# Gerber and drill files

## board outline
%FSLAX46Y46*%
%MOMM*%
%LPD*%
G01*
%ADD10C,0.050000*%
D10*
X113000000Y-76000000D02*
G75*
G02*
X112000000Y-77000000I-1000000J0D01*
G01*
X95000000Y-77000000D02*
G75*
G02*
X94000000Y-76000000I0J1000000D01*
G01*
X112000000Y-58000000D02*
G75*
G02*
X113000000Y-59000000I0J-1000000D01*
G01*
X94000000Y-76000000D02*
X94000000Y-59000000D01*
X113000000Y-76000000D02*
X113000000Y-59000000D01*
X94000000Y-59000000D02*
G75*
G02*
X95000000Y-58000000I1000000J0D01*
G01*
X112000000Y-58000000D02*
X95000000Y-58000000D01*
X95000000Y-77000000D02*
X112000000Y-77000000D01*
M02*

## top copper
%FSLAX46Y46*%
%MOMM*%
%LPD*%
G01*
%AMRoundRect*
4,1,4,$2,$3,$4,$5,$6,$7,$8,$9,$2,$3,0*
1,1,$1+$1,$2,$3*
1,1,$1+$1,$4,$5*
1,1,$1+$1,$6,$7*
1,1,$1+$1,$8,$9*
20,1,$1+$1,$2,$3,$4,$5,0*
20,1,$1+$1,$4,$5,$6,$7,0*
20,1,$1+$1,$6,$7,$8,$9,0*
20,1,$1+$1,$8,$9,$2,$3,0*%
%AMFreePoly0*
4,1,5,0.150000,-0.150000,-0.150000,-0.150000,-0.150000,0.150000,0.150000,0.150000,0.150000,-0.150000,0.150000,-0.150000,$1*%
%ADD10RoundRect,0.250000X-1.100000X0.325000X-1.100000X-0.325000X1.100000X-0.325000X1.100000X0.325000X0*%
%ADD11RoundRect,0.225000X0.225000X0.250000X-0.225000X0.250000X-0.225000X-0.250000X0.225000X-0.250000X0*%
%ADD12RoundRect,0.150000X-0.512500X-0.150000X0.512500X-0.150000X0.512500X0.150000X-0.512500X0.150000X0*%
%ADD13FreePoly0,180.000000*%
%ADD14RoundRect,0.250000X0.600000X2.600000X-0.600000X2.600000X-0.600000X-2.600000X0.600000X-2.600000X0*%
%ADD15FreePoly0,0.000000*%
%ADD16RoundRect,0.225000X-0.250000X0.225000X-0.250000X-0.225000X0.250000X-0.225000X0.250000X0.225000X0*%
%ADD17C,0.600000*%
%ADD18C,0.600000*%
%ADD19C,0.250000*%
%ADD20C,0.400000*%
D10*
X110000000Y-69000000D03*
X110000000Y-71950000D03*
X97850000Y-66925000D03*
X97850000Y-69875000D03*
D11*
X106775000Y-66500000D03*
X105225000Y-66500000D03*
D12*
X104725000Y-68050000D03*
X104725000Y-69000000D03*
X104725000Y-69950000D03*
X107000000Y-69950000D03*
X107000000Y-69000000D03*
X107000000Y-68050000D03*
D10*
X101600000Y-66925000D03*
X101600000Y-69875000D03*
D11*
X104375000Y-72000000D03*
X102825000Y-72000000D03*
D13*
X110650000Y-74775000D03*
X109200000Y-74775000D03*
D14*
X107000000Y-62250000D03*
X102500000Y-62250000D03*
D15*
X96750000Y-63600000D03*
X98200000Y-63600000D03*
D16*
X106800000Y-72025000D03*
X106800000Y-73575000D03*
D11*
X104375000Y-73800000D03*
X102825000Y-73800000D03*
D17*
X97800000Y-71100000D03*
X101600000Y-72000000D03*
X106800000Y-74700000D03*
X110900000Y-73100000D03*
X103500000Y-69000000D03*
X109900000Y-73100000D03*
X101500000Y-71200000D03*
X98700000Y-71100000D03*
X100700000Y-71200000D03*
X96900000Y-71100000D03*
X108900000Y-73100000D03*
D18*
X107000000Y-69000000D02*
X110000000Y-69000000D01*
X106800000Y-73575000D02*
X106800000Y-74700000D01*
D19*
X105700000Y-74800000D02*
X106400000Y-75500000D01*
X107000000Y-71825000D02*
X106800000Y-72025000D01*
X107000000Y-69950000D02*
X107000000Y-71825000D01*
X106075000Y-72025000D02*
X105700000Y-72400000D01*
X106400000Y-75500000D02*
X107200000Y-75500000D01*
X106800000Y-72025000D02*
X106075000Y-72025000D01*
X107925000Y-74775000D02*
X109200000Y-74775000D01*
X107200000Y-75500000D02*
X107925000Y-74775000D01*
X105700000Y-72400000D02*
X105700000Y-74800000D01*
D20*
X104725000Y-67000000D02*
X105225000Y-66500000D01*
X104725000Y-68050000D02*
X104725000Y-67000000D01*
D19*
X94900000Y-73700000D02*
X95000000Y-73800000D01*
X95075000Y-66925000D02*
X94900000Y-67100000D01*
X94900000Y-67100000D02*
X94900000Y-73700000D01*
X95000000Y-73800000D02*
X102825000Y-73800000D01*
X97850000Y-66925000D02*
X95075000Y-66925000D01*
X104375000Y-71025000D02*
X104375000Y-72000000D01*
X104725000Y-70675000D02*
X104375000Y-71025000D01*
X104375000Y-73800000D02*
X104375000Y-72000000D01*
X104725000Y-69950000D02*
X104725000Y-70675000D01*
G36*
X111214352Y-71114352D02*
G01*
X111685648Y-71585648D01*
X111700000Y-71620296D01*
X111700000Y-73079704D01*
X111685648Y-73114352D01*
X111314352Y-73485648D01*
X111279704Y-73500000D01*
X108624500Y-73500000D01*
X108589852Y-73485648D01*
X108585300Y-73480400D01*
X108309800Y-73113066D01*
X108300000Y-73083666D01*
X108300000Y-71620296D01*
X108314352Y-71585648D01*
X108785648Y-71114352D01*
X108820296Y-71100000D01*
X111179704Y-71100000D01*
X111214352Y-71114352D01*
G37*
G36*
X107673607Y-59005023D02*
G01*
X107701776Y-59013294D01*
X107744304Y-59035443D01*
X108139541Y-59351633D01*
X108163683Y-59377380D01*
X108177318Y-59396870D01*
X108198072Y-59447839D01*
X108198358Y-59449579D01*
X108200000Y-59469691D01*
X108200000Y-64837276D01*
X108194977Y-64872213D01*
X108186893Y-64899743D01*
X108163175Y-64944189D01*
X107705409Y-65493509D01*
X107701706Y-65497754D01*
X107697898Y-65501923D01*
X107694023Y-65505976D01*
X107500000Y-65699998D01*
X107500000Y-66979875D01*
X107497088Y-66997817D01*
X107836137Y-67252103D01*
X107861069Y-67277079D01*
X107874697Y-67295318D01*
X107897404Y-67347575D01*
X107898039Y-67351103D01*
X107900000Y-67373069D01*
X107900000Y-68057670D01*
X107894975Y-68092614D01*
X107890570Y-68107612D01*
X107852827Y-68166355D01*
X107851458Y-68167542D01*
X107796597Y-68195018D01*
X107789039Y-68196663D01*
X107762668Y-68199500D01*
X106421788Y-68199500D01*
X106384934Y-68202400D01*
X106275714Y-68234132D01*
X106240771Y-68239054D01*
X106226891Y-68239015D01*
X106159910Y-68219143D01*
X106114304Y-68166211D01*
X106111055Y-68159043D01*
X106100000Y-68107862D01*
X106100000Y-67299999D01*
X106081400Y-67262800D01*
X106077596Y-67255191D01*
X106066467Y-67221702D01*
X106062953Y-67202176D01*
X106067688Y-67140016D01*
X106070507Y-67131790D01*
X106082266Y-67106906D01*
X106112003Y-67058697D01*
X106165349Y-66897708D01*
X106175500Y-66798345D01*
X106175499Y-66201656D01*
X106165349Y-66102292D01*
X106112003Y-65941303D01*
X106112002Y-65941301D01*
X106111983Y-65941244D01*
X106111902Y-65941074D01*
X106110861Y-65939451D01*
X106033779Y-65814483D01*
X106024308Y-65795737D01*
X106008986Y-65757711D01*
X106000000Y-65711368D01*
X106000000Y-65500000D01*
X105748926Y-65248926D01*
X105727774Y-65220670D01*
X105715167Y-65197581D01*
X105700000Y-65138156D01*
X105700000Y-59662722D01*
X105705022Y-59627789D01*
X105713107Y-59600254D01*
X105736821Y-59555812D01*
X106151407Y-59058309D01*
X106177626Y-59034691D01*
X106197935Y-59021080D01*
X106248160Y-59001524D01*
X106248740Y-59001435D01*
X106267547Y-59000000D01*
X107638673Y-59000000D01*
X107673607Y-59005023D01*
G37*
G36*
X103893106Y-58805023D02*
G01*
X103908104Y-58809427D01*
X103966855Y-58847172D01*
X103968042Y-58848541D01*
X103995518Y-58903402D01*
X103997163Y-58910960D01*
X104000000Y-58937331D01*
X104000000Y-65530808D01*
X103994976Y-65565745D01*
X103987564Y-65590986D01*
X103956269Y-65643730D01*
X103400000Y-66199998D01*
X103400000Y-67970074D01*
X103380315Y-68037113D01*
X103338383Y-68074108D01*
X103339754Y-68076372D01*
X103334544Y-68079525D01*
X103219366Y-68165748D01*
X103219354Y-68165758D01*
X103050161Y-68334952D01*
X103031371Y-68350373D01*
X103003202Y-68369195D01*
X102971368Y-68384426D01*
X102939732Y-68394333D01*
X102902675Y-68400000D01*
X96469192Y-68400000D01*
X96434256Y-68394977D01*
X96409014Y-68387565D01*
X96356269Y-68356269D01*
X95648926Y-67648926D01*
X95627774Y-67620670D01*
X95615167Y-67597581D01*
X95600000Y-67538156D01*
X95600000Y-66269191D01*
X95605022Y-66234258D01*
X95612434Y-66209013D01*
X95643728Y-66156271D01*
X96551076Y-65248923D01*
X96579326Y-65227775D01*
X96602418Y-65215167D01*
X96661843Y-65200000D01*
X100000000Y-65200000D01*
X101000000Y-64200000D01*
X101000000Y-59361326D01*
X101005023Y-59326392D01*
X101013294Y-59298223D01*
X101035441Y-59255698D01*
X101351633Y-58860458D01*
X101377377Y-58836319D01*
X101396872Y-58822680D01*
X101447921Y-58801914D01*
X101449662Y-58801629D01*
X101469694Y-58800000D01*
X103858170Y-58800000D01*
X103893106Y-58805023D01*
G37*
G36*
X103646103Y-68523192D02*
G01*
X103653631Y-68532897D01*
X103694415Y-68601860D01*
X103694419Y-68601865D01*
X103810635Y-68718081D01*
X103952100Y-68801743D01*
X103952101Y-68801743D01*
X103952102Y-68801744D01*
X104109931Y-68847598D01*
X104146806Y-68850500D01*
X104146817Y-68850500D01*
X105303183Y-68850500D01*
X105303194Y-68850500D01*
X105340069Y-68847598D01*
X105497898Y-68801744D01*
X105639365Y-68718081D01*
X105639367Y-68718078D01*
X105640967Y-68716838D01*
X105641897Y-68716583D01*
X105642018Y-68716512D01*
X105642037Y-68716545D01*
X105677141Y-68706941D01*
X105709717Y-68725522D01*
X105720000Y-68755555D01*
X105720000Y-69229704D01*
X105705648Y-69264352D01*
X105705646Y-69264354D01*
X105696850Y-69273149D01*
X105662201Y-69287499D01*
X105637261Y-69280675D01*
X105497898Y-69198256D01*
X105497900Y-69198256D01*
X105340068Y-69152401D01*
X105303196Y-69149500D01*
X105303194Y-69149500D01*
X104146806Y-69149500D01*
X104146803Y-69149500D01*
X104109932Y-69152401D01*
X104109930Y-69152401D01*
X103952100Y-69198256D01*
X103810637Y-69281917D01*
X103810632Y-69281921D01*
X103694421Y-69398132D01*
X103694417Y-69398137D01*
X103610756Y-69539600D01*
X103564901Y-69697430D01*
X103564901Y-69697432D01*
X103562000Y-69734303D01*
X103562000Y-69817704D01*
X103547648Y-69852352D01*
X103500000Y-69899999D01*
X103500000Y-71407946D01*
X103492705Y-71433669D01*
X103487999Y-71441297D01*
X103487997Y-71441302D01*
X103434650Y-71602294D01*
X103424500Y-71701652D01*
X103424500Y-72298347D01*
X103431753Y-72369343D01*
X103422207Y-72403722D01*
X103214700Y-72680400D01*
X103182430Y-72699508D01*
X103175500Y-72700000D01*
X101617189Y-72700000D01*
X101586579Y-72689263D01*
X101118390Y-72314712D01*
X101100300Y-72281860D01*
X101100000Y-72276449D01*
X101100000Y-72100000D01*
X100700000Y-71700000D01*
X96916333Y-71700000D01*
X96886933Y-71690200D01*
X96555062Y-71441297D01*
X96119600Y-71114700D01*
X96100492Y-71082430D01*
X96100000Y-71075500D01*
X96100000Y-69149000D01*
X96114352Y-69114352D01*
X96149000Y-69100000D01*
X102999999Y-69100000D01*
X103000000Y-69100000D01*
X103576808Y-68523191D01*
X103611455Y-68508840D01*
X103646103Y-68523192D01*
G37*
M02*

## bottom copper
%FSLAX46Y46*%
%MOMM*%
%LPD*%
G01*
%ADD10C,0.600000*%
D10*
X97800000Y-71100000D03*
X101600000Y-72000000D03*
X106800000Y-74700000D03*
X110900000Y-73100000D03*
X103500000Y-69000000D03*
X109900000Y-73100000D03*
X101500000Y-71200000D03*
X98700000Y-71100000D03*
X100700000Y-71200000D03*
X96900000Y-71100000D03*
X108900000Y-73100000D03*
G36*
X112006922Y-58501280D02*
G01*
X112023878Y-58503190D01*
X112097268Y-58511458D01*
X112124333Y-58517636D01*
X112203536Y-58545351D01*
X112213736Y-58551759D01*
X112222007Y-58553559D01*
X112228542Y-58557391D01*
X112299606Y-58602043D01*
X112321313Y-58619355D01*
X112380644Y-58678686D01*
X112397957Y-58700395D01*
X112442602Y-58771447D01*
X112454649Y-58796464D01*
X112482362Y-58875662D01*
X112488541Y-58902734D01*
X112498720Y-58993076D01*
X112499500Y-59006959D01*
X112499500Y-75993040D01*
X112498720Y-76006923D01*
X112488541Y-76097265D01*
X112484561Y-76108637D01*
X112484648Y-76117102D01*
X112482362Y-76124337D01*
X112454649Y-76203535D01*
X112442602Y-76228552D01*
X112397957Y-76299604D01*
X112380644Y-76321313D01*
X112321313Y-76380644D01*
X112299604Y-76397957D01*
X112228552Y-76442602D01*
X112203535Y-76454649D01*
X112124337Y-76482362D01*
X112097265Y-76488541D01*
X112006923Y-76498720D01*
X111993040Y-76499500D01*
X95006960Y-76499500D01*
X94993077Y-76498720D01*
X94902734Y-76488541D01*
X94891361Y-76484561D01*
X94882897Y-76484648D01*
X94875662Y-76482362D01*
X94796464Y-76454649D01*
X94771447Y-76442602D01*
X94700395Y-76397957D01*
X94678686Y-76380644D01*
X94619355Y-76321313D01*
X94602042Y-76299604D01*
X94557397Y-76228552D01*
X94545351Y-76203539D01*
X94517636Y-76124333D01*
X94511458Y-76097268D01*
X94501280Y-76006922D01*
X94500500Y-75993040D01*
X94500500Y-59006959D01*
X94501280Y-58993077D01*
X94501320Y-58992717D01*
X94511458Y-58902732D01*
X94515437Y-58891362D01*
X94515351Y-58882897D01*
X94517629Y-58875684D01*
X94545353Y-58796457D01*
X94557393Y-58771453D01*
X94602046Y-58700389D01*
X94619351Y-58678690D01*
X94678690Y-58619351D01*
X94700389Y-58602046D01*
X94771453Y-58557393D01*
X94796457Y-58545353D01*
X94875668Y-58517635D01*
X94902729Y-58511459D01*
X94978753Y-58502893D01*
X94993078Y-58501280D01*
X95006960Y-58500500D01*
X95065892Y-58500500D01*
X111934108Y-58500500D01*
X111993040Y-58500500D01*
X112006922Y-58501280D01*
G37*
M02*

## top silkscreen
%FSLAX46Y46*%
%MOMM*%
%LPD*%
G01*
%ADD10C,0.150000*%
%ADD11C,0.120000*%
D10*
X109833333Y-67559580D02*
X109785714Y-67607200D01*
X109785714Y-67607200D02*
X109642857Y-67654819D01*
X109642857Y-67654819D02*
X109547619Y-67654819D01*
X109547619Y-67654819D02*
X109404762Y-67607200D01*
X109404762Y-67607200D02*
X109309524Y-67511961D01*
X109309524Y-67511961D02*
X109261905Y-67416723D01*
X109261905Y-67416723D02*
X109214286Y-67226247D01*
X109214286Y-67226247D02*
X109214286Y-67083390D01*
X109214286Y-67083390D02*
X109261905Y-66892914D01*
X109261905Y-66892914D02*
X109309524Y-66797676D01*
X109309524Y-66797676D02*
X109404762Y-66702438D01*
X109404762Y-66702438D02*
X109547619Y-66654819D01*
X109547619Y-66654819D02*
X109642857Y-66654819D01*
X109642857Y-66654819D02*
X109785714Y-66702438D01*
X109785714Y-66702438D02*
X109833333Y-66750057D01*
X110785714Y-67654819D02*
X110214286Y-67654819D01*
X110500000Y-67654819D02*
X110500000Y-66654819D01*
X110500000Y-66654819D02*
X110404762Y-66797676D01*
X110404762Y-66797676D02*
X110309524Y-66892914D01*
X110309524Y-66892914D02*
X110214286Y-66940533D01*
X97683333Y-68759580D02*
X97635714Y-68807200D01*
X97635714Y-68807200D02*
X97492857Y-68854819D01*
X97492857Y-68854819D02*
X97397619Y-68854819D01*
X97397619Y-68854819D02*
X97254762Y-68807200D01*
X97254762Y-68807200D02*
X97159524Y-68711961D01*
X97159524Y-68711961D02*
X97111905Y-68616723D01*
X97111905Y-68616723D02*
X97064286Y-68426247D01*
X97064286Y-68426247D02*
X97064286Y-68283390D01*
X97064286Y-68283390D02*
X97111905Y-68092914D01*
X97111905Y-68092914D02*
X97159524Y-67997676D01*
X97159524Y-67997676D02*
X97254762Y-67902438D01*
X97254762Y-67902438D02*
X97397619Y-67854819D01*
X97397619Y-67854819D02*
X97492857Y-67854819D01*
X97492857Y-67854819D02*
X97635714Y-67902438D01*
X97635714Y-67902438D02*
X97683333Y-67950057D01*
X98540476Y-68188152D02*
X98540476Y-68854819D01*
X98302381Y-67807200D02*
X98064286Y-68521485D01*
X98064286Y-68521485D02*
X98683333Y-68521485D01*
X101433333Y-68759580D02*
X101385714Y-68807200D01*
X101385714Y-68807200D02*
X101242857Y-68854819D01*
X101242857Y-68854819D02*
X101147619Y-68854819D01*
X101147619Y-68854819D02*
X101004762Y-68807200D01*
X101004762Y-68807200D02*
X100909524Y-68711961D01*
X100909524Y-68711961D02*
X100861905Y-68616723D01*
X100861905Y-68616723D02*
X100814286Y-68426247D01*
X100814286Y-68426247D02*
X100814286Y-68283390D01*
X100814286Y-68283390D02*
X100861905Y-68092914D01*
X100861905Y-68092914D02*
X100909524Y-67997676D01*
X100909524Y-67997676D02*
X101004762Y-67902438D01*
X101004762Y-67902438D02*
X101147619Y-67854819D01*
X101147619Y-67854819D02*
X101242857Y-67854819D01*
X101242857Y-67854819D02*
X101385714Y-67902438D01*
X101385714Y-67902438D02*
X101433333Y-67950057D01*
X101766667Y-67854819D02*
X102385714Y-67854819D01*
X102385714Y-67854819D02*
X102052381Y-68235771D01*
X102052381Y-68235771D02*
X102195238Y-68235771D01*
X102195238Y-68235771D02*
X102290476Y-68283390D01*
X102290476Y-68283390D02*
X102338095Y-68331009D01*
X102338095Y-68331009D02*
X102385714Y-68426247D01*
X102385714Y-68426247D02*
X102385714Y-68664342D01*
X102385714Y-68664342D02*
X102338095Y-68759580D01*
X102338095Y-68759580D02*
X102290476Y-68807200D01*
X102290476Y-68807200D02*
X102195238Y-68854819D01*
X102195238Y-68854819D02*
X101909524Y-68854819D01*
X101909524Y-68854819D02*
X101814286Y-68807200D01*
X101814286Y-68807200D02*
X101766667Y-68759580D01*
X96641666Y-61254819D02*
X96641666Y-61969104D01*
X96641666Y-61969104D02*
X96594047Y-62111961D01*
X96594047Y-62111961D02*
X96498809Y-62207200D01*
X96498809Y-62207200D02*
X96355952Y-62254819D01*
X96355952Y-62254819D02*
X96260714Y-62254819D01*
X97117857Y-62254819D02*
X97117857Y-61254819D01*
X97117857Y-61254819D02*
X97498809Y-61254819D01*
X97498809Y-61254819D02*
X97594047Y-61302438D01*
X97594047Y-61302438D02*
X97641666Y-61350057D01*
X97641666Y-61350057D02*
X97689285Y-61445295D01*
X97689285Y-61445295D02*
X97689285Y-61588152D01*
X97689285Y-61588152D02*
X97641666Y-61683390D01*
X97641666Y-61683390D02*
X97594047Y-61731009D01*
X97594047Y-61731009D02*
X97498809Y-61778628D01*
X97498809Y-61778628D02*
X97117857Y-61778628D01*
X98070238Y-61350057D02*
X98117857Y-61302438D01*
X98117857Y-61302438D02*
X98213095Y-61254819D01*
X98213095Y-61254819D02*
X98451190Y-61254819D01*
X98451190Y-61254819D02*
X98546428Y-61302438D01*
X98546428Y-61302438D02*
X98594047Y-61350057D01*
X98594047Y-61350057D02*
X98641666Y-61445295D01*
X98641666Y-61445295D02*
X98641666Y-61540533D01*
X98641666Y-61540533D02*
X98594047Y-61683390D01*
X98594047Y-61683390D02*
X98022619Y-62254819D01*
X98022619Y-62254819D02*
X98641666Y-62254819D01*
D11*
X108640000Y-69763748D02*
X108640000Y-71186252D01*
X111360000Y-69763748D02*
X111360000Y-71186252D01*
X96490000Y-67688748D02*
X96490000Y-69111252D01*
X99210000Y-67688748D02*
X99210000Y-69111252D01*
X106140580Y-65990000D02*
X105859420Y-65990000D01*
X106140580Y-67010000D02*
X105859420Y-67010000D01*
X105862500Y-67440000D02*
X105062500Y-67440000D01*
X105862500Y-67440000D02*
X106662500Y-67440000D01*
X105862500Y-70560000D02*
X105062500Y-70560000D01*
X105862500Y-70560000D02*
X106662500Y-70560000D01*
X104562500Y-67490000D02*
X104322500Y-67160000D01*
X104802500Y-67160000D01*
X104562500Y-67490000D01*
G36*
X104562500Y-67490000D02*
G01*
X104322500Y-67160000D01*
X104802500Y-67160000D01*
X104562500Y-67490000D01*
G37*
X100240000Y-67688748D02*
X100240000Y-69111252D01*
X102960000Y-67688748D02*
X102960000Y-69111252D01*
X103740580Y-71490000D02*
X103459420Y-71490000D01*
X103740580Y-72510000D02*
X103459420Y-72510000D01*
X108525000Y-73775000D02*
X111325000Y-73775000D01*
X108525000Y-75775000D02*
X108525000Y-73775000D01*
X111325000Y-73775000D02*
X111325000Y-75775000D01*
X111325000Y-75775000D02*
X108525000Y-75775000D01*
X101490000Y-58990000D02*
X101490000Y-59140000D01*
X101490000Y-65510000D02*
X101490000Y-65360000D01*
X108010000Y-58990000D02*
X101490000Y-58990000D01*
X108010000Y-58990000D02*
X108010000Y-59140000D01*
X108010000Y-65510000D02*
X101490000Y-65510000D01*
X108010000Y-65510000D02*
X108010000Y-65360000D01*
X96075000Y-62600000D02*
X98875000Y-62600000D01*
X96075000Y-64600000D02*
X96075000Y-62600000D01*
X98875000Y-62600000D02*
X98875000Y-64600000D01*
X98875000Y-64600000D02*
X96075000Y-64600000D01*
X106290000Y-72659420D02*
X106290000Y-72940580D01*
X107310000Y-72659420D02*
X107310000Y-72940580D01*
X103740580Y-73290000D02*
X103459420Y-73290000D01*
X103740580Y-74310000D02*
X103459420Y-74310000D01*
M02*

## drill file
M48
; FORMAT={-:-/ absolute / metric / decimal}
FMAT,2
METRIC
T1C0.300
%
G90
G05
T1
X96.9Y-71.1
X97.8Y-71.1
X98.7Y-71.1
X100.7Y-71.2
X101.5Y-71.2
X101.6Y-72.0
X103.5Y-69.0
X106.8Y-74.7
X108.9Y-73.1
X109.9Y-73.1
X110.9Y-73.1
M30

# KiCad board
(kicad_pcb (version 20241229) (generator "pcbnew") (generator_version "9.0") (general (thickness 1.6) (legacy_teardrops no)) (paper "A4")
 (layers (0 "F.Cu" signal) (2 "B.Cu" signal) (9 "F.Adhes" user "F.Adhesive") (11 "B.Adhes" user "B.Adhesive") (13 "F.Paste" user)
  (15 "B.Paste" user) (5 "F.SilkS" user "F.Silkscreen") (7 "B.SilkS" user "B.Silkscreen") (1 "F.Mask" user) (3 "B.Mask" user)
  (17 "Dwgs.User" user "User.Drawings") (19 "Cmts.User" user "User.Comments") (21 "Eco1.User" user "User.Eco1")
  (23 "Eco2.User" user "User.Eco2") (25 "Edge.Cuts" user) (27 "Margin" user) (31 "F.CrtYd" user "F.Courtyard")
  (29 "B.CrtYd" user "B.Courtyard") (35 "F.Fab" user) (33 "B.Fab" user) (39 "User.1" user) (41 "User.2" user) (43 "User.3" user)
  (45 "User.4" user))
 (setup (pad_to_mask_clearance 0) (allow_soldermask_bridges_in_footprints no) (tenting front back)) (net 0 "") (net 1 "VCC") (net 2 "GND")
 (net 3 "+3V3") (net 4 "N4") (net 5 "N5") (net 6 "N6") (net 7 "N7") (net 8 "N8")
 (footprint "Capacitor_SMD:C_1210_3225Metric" (layer "F.Cu") (at 110 70.475 -90)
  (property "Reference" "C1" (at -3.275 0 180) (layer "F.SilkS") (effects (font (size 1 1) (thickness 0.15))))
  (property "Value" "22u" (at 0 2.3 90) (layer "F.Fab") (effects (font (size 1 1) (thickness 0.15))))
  (fp_line (start -0.711252 1.36) (end 0.711252 1.36) (stroke (width 0.12) (type solid)) (layer "F.SilkS"))
  (fp_line (start -0.711252 -1.36) (end 0.711252 -1.36) (stroke (width 0.12) (type solid)) (layer "F.SilkS"))
  (pad "1" smd roundrect (at -1.475 0 270) (size 1.15 2.7) (layers "F.Cu" "F.Mask" "F.Paste") (roundrect_rratio 0.217391) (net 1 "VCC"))
  (pad "2" smd roundrect (at 1.475 0 270) (size 1.15 2.7) (layers "F.Cu" "F.Mask" "F.Paste") (roundrect_rratio 0.217391) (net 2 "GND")))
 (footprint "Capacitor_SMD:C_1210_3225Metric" (layer "F.Cu") (at 97.85 68.4 -90)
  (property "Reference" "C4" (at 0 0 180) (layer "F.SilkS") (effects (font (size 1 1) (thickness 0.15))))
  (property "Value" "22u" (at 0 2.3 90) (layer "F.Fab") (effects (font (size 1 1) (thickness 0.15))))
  (fp_line (start -0.711252 1.36) (end 0.711252 1.36) (stroke (width 0.12) (type solid)) (layer "F.SilkS"))
  (fp_line (start -0.711252 -1.36) (end 0.711252 -1.36) (stroke (width 0.12) (type solid)) (layer "F.SilkS"))
  (pad "1" smd roundrect (at -1.475 0 270) (size 1.15 2.7) (layers "F.Cu" "F.Mask" "F.Paste") (roundrect_rratio 0.217391) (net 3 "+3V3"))
  (pad "2" smd roundrect (at 1.475 0 270) (size 1.15 2.7) (layers "F.Cu" "F.Mask" "F.Paste") (roundrect_rratio 0.217391) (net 2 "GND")))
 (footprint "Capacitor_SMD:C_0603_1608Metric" (layer "F.Cu") (at 106 66.5 180)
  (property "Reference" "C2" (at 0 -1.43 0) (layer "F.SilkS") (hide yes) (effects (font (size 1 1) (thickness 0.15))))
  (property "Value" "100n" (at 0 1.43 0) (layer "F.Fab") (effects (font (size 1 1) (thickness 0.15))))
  (fp_line (start -0.14058 0.51) (end 0.14058 0.51) (stroke (width 0.12) (type solid)) (layer "F.SilkS"))
  (fp_line (start -0.14058 -0.51) (end 0.14058 -0.51) (stroke (width 0.12) (type solid)) (layer "F.SilkS"))
  (pad "1" smd roundrect (at -0.775 0 180) (size 0.9 0.95) (layers "F.Cu" "F.Mask" "F.Paste") (roundrect_rratio 0.25) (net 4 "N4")
   (thermal_bridge_width 0.3) (thermal_gap 0.3))
  (pad "2" smd roundrect (at 0.775 0 180) (size 0.9 0.95) (layers "F.Cu" "F.Mask" "F.Paste") (roundrect_rratio 0.25) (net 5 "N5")))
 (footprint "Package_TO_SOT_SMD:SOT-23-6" (layer "F.Cu") (at 105.8625 69)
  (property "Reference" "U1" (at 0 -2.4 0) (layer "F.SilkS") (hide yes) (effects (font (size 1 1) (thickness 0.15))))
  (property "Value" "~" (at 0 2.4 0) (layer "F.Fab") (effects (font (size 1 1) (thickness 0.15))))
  (fp_line (start 0 -1.56) (end -0.8 -1.56) (stroke (width 0.12) (type solid)) (layer "F.SilkS"))
  (fp_line (start 0 -1.56) (end 0.8 -1.56) (stroke (width 0.12) (type solid)) (layer "F.SilkS"))
  (fp_line (start 0 1.56) (end -0.8 1.56) (stroke (width 0.12) (type solid)) (layer "F.SilkS"))
  (fp_line (start 0 1.56) (end 0.8 1.56) (stroke (width 0.12) (type solid)) (layer "F.SilkS"))
  (fp_poly
   (pts (xy -1.3 -1.51) (xy -1.54 -1.84) (xy -1.06 -1.84) (xy -1.3 -1.51)) (stroke (width 0.12) (type solid)) (fill yes) (layer "F.SilkS"))
  (pad "1" smd roundrect (at -1.1375 -0.95) (size 1.325 0.6) (layers "F.Cu" "F.Mask" "F.Paste") (roundrect_rratio 0.25) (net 5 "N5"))
  (pad "2" smd roundrect (at -1.1375 0) (size 1.325 0.6) (layers "F.Cu" "F.Mask" "F.Paste") (roundrect_rratio 0.25) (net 2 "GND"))
  (pad "3" smd roundrect (at -1.1375 0.95) (size 1.325 0.6) (layers "F.Cu" "F.Mask" "F.Paste") (roundrect_rratio 0.25) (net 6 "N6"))
  (pad "4" smd roundrect (at 1.1375 0.95) (size 1.325 0.6) (layers "F.Cu" "F.Mask" "F.Paste") (roundrect_rratio 0.25) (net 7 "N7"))
  (pad "5" smd roundrect (at 1.1375 0) (size 1.325 0.6) (layers "F.Cu" "F.Mask" "F.Paste") (roundrect_rratio 0.25) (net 1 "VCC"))
  (pad "6" smd roundrect (at 1.1375 -0.95) (size 1.325 0.6) (layers "F.Cu" "F.Mask" "F.Paste") (roundrect_rratio 0.25) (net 4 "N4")))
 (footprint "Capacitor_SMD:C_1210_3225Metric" (layer "F.Cu") (at 101.6 68.4 -90)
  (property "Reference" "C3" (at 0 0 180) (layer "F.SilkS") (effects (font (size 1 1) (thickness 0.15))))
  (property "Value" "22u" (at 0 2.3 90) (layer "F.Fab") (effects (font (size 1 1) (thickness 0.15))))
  (fp_line (start -0.711252 1.36) (end 0.711252 1.36) (stroke (width 0.12) (type solid)) (layer "F.SilkS"))
  (fp_line (start -0.711252 -1.36) (end 0.711252 -1.36) (stroke (width 0.12) (type solid)) (layer "F.SilkS"))
  (pad "1" smd roundrect (at -1.475 0 270) (size 1.15 2.7) (layers "F.Cu" "F.Mask" "F.Paste") (roundrect_rratio 0.217391) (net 3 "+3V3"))
  (pad "2" smd roundrect (at 1.475 0 270) (size 1.15 2.7) (layers "F.Cu" "F.Mask" "F.Paste") (roundrect_rratio 0.217391) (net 2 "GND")))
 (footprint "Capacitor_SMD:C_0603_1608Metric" (layer "F.Cu") (at 103.6 72 180)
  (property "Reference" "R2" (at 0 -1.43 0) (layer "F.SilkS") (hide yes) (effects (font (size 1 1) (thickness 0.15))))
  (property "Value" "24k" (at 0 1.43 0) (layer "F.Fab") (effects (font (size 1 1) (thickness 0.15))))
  (fp_line (start -0.14058 0.51) (end 0.14058 0.51) (stroke (width 0.12) (type solid)) (layer "F.SilkS"))
  (fp_line (start -0.14058 -0.51) (end 0.14058 -0.51) (stroke (width 0.12) (type solid)) (layer "F.SilkS"))
  (pad "1" smd roundrect (at -0.775 0 180) (size 0.9 0.95) (layers "F.Cu" "F.Mask" "F.Paste") (roundrect_rratio 0.25) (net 6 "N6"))
  (pad "2" smd roundrect (at 0.775 0 180) (size 0.9 0.95) (layers "F.Cu" "F.Mask" "F.Paste") (roundrect_rratio 0.25) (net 2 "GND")
   (thermal_bridge_width 0.2) (thermal_gap 0.2)))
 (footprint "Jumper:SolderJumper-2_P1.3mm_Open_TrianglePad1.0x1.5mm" (layer "F.Cu") (at 109.925 74.775 180)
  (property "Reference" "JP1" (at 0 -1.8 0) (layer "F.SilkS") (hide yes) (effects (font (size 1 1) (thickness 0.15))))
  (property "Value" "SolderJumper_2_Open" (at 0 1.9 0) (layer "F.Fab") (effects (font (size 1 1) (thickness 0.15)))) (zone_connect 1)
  (fp_line (start 1.4 1) (end -1.4 1) (stroke (width 0.12) (type solid)) (layer "F.SilkS"))
  (fp_line (start 1.4 -1) (end 1.4 1) (stroke (width 0.12) (type solid)) (layer "F.SilkS"))
  (fp_line (start -1.4 1) (end -1.4 -1) (stroke (width 0.12) (type solid)) (layer "F.SilkS"))
  (fp_line (start -1.4 -1) (end 1.4 -1) (stroke (width 0.12) (type solid)) (layer "F.SilkS"))
  (pad "1" smd custom (at -0.725 0 180) (size 0.3 0.3) (layers "F.Cu" "F.Mask") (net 1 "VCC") (zone_connect 2) (thermal_bridge_angle 45)
   (options (clearance outline) (anchor rect)) (primitives))
  (pad "2" smd custom (at 0.725 0 180) (size 0.3 0.3) (layers "F.Cu" "F.Mask") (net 7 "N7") (zone_connect 2) (thermal_bridge_angle 45)
   (options (clearance outline) (anchor rect)) (primitives)))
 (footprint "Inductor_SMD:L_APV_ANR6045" (layer "F.Cu") (at 104.75 62.25 180)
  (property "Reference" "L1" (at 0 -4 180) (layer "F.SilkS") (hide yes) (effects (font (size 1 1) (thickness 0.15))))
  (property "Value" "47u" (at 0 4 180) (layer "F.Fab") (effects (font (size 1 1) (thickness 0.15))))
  (fp_line (start 3.26 3.26) (end 3.26 3.11) (stroke (width 0.12) (type solid)) (layer "F.SilkS"))
  (fp_line (start 3.26 -3.26) (end 3.26 -3.11) (stroke (width 0.12) (type solid)) (layer "F.SilkS"))
  (fp_line (start -3.26 3.26) (end 3.26 3.26) (stroke (width 0.12) (type solid)) (layer "F.SilkS"))
  (fp_line (start -3.26 3.26) (end -3.26 3.11) (stroke (width 0.12) (type solid)) (layer "F.SilkS"))
  (fp_line (start -3.26 -3.26) (end 3.26 -3.26) (stroke (width 0.12) (type solid)) (layer "F.SilkS"))
  (fp_line (start -3.26 -3.26) (end -3.26 -3.11) (stroke (width 0.12) (type solid)) (layer "F.SilkS"))
  (pad "1" smd roundrect (at -2.25 0 180) (size 1.7 5.7) (layers "F.Cu" "F.Mask" "F.Paste") (roundrect_rratio 0.147059) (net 4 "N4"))
  (pad "2" smd roundrect (at 2.25 0 180) (size 1.7 5.7) (layers "F.Cu" "F.Mask" "F.Paste") (roundrect_rratio 0.147059) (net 3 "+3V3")))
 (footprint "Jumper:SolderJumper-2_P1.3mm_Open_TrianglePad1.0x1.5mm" (layer "F.Cu") (at 97.475 63.6)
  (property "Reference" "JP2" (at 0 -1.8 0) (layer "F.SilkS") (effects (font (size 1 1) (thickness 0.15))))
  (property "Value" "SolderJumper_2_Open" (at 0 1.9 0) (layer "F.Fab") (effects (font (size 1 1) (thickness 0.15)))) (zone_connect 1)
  (fp_line (start -1.4 -1) (end 1.4 -1) (stroke (width 0.12) (type solid)) (layer "F.SilkS"))
  (fp_line (start -1.4 1) (end -1.4 -1) (stroke (width 0.12) (type solid)) (layer "F.SilkS"))
  (fp_line (start 1.4 -1) (end 1.4 1) (stroke (width 0.12) (type solid)) (layer "F.SilkS"))
  (fp_line (start 1.4 1) (end -1.4 1) (stroke (width 0.12) (type solid)) (layer "F.SilkS"))
  (pad "1" smd custom (at -0.725 0) (size 0.3 0.3) (layers "F.Cu" "F.Mask") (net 3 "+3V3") (zone_connect 2) (thermal_bridge_angle 45)
   (options (clearance outline) (anchor rect)) (primitives))
  (pad "2" smd custom (at 0.725 0) (size 0.3 0.3) (layers "F.Cu" "F.Mask") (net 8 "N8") (zone_connect 2) (thermal_bridge_angle 45)
   (options (clearance outline) (anchor rect)) (primitives)))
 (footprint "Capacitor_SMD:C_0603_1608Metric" (layer "F.Cu") (at 106.8 72.8 -90)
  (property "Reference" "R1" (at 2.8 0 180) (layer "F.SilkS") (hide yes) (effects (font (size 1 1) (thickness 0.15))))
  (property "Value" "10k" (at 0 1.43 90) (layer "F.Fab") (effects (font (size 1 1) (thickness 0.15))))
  (fp_line (start -0.14058 0.51) (end 0.14058 0.51) (stroke (width 0.12) (type solid)) (layer "F.SilkS"))
  (fp_line (start -0.14058 -0.51) (end 0.14058 -0.51) (stroke (width 0.12) (type solid)) (layer "F.SilkS"))
  (pad "1" smd roundrect (at -0.775 0 270) (size 0.9 0.95) (layers "F.Cu" "F.Mask" "F.Paste") (roundrect_rratio 0.25) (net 7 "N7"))
  (pad "2" smd roundrect (at 0.775 0 270) (size 0.9 0.95) (layers "F.Cu" "F.Mask" "F.Paste") (roundrect_rratio 0.25) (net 2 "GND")))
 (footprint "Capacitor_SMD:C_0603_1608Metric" (layer "F.Cu") (at 103.6 73.8 180)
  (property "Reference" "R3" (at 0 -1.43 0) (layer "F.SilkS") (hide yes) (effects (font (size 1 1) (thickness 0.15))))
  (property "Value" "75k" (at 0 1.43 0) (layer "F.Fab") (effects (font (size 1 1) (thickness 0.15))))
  (fp_line (start -0.14058 0.51) (end 0.14058 0.51) (stroke (width 0.12) (type solid)) (layer "F.SilkS"))
  (fp_line (start -0.14058 -0.51) (end 0.14058 -0.51) (stroke (width 0.12) (type solid)) (layer "F.SilkS"))
  (pad "1" smd roundrect (at -0.775 0 180) (size 0.9 0.95) (layers "F.Cu" "F.Mask" "F.Paste") (roundrect_rratio 0.25) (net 6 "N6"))
  (pad "2" smd roundrect (at 0.775 0 180) (size 0.9 0.95) (layers "F.Cu" "F.Mask" "F.Paste") (roundrect_rratio 0.25) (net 3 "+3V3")))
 (gr_arc (start 113 76) (mid 112.707107 76.707107) (end 112 77) (stroke (width 0.05) (type default)) (layer "Edge.Cuts"))
 (gr_arc (start 95 77) (mid 94.292893 76.707107) (end 94 76) (stroke (width 0.05) (type default)) (layer "Edge.Cuts"))
 (gr_arc (start 112 58) (mid 112.707107 58.292893) (end 113 59) (stroke (width 0.05) (type default)) (layer "Edge.Cuts"))
 (gr_line (start 94 76) (end 94 59) (stroke (width 0.05) (type default)) (layer "Edge.Cuts"))
 (gr_line (start 113 76) (end 113 59) (stroke (width 0.05) (type default)) (layer "Edge.Cuts"))
 (gr_arc (start 94 59) (mid 94.292893 58.292893) (end 95 58) (stroke (width 0.05) (type default)) (layer "Edge.Cuts"))
 (gr_line (start 112 58) (end 95 58) (stroke (width 0.05) (type default)) (layer "Edge.Cuts"))
 (gr_line (start 95 77) (end 112 77) (stroke (width 0.05) (type default)) (layer "Edge.Cuts"))
 (segment (start 107 69) (end 110 69) (width 0.6) (layer "F.Cu") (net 1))
 (segment (start 106.8 73.575) (end 106.8 74.7) (width 0.6) (layer "F.Cu") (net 2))
 (via (at 97.8 71.1) (size 0.6) (drill 0.3) (layers "F.Cu" "B.Cu") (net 2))
 (via (at 101.6 72) (size 0.6) (drill 0.3) (layers "F.Cu" "B.Cu") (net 2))
 (via (at 106.8 74.7) (size 0.6) (drill 0.3) (layers "F.Cu" "B.Cu") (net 2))
 (via (at 110.9 73.1) (size 0.6) (drill 0.3) (layers "F.Cu" "B.Cu") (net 2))
 (via (at 103.5 69) (size 0.6) (drill 0.3) (layers "F.Cu" "B.Cu") (free yes) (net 2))
 (via (at 109.9 73.1) (size 0.6) (drill 0.3) (layers "F.Cu" "B.Cu") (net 2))
 (via (at 101.5 71.2) (size 0.6) (drill 0.3) (layers "F.Cu" "B.Cu") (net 2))
 (via (at 98.7 71.1) (size 0.6) (drill 0.3) (layers "F.Cu" "B.Cu") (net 2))
 (via (at 100.7 71.2) (size 0.6) (drill 0.3) (layers "F.Cu" "B.Cu") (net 2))
 (via (at 96.9 71.1) (size 0.6) (drill 0.3) (layers "F.Cu" "B.Cu") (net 2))
 (via (at 108.9 73.1) (size 0.6) (drill 0.3) (layers "F.Cu" "B.Cu") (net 2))
 (segment (start 105.7 74.8) (end 106.4 75.5) (width 0.25) (layer "F.Cu") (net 7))
 (segment (start 107 71.825) (end 106.8 72.025) (width 0.25) (layer "F.Cu") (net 7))
 (segment (start 107 69.95) (end 107 71.825) (width 0.25) (layer "F.Cu") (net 7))
 (segment (start 106.075 72.025) (end 105.7 72.4) (width 0.25) (layer "F.Cu") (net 7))
 (segment (start 106.4 75.5) (end 107.2 75.5) (width 0.25) (layer "F.Cu") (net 7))
 (segment (start 106.8 72.025) (end 106.075 72.025) (width 0.25) (layer "F.Cu") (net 7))
 (segment (start 107.925 74.775) (end 109.2 74.775) (width 0.25) (layer "F.Cu") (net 7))
 (segment (start 107.2 75.5) (end 107.925 74.775) (width 0.25) (layer "F.Cu") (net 7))
 (segment (start 105.7 72.4) (end 105.7 74.8) (width 0.25) (layer "F.Cu") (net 7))
 (segment (start 104.725 67) (end 105.225 66.5) (width 0.4) (layer "F.Cu") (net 5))
 (segment (start 104.725 68.05) (end 104.725 67) (width 0.4) (layer "F.Cu") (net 5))
 (segment (start 94.9 73.7) (end 95 73.8) (width 0.25) (layer "F.Cu") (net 3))
 (segment (start 95.075 66.925) (end 94.9 67.1) (width 0.25) (layer "F.Cu") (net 3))
 (segment (start 94.9 67.1) (end 94.9 73.7) (width 0.25) (layer "F.Cu") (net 3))
 (segment (start 95 73.8) (end 102.825 73.8) (width 0.25) (layer "F.Cu") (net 3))
 (segment (start 97.85 66.925) (end 95.075 66.925) (width 0.25) (layer "F.Cu") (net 3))
 (segment (start 104.375 71.025) (end 104.375 72) (width 0.25) (layer "F.Cu") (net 6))
 (segment (start 104.725 70.675) (end 104.375 71.025) (width 0.25) (layer "F.Cu") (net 6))
 (segment (start 104.375 73.8) (end 104.375 72) (width 0.25) (layer "F.Cu") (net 6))
 (segment (start 104.725 69.95) (end 104.725 70.675) (width 0.25) (layer "F.Cu") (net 6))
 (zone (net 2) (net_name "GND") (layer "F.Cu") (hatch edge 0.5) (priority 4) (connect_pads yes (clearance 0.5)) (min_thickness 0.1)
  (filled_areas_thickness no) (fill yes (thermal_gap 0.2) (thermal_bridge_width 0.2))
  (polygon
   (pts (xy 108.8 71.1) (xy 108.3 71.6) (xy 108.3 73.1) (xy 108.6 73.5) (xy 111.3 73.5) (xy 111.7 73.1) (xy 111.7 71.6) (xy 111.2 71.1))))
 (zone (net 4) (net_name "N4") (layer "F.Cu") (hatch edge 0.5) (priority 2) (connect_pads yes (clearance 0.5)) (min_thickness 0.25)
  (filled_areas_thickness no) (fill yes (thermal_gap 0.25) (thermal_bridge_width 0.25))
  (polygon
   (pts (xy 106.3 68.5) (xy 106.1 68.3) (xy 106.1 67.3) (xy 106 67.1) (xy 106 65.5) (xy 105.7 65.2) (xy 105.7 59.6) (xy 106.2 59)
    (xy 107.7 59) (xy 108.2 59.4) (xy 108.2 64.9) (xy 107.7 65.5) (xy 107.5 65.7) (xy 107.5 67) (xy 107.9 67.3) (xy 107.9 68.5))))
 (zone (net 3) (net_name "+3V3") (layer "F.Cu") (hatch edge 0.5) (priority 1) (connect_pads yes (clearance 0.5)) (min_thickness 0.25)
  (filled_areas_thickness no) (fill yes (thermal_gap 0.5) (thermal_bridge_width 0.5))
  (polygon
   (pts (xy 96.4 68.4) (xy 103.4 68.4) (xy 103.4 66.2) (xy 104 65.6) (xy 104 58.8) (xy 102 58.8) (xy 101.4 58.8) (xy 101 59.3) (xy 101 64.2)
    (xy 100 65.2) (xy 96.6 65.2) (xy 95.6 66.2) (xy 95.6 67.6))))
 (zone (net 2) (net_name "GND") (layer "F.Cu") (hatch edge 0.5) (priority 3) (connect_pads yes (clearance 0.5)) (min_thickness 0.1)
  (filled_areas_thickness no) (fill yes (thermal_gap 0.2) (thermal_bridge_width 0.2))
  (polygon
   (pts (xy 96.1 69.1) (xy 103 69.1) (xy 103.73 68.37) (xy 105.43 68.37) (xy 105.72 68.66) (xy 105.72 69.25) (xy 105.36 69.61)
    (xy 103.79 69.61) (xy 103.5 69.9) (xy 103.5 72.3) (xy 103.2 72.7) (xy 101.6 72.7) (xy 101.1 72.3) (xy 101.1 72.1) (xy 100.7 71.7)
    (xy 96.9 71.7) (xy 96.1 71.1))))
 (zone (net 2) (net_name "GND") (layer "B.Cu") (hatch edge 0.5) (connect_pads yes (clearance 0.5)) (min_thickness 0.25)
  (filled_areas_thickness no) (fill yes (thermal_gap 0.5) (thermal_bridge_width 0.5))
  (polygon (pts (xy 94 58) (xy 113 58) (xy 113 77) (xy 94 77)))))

